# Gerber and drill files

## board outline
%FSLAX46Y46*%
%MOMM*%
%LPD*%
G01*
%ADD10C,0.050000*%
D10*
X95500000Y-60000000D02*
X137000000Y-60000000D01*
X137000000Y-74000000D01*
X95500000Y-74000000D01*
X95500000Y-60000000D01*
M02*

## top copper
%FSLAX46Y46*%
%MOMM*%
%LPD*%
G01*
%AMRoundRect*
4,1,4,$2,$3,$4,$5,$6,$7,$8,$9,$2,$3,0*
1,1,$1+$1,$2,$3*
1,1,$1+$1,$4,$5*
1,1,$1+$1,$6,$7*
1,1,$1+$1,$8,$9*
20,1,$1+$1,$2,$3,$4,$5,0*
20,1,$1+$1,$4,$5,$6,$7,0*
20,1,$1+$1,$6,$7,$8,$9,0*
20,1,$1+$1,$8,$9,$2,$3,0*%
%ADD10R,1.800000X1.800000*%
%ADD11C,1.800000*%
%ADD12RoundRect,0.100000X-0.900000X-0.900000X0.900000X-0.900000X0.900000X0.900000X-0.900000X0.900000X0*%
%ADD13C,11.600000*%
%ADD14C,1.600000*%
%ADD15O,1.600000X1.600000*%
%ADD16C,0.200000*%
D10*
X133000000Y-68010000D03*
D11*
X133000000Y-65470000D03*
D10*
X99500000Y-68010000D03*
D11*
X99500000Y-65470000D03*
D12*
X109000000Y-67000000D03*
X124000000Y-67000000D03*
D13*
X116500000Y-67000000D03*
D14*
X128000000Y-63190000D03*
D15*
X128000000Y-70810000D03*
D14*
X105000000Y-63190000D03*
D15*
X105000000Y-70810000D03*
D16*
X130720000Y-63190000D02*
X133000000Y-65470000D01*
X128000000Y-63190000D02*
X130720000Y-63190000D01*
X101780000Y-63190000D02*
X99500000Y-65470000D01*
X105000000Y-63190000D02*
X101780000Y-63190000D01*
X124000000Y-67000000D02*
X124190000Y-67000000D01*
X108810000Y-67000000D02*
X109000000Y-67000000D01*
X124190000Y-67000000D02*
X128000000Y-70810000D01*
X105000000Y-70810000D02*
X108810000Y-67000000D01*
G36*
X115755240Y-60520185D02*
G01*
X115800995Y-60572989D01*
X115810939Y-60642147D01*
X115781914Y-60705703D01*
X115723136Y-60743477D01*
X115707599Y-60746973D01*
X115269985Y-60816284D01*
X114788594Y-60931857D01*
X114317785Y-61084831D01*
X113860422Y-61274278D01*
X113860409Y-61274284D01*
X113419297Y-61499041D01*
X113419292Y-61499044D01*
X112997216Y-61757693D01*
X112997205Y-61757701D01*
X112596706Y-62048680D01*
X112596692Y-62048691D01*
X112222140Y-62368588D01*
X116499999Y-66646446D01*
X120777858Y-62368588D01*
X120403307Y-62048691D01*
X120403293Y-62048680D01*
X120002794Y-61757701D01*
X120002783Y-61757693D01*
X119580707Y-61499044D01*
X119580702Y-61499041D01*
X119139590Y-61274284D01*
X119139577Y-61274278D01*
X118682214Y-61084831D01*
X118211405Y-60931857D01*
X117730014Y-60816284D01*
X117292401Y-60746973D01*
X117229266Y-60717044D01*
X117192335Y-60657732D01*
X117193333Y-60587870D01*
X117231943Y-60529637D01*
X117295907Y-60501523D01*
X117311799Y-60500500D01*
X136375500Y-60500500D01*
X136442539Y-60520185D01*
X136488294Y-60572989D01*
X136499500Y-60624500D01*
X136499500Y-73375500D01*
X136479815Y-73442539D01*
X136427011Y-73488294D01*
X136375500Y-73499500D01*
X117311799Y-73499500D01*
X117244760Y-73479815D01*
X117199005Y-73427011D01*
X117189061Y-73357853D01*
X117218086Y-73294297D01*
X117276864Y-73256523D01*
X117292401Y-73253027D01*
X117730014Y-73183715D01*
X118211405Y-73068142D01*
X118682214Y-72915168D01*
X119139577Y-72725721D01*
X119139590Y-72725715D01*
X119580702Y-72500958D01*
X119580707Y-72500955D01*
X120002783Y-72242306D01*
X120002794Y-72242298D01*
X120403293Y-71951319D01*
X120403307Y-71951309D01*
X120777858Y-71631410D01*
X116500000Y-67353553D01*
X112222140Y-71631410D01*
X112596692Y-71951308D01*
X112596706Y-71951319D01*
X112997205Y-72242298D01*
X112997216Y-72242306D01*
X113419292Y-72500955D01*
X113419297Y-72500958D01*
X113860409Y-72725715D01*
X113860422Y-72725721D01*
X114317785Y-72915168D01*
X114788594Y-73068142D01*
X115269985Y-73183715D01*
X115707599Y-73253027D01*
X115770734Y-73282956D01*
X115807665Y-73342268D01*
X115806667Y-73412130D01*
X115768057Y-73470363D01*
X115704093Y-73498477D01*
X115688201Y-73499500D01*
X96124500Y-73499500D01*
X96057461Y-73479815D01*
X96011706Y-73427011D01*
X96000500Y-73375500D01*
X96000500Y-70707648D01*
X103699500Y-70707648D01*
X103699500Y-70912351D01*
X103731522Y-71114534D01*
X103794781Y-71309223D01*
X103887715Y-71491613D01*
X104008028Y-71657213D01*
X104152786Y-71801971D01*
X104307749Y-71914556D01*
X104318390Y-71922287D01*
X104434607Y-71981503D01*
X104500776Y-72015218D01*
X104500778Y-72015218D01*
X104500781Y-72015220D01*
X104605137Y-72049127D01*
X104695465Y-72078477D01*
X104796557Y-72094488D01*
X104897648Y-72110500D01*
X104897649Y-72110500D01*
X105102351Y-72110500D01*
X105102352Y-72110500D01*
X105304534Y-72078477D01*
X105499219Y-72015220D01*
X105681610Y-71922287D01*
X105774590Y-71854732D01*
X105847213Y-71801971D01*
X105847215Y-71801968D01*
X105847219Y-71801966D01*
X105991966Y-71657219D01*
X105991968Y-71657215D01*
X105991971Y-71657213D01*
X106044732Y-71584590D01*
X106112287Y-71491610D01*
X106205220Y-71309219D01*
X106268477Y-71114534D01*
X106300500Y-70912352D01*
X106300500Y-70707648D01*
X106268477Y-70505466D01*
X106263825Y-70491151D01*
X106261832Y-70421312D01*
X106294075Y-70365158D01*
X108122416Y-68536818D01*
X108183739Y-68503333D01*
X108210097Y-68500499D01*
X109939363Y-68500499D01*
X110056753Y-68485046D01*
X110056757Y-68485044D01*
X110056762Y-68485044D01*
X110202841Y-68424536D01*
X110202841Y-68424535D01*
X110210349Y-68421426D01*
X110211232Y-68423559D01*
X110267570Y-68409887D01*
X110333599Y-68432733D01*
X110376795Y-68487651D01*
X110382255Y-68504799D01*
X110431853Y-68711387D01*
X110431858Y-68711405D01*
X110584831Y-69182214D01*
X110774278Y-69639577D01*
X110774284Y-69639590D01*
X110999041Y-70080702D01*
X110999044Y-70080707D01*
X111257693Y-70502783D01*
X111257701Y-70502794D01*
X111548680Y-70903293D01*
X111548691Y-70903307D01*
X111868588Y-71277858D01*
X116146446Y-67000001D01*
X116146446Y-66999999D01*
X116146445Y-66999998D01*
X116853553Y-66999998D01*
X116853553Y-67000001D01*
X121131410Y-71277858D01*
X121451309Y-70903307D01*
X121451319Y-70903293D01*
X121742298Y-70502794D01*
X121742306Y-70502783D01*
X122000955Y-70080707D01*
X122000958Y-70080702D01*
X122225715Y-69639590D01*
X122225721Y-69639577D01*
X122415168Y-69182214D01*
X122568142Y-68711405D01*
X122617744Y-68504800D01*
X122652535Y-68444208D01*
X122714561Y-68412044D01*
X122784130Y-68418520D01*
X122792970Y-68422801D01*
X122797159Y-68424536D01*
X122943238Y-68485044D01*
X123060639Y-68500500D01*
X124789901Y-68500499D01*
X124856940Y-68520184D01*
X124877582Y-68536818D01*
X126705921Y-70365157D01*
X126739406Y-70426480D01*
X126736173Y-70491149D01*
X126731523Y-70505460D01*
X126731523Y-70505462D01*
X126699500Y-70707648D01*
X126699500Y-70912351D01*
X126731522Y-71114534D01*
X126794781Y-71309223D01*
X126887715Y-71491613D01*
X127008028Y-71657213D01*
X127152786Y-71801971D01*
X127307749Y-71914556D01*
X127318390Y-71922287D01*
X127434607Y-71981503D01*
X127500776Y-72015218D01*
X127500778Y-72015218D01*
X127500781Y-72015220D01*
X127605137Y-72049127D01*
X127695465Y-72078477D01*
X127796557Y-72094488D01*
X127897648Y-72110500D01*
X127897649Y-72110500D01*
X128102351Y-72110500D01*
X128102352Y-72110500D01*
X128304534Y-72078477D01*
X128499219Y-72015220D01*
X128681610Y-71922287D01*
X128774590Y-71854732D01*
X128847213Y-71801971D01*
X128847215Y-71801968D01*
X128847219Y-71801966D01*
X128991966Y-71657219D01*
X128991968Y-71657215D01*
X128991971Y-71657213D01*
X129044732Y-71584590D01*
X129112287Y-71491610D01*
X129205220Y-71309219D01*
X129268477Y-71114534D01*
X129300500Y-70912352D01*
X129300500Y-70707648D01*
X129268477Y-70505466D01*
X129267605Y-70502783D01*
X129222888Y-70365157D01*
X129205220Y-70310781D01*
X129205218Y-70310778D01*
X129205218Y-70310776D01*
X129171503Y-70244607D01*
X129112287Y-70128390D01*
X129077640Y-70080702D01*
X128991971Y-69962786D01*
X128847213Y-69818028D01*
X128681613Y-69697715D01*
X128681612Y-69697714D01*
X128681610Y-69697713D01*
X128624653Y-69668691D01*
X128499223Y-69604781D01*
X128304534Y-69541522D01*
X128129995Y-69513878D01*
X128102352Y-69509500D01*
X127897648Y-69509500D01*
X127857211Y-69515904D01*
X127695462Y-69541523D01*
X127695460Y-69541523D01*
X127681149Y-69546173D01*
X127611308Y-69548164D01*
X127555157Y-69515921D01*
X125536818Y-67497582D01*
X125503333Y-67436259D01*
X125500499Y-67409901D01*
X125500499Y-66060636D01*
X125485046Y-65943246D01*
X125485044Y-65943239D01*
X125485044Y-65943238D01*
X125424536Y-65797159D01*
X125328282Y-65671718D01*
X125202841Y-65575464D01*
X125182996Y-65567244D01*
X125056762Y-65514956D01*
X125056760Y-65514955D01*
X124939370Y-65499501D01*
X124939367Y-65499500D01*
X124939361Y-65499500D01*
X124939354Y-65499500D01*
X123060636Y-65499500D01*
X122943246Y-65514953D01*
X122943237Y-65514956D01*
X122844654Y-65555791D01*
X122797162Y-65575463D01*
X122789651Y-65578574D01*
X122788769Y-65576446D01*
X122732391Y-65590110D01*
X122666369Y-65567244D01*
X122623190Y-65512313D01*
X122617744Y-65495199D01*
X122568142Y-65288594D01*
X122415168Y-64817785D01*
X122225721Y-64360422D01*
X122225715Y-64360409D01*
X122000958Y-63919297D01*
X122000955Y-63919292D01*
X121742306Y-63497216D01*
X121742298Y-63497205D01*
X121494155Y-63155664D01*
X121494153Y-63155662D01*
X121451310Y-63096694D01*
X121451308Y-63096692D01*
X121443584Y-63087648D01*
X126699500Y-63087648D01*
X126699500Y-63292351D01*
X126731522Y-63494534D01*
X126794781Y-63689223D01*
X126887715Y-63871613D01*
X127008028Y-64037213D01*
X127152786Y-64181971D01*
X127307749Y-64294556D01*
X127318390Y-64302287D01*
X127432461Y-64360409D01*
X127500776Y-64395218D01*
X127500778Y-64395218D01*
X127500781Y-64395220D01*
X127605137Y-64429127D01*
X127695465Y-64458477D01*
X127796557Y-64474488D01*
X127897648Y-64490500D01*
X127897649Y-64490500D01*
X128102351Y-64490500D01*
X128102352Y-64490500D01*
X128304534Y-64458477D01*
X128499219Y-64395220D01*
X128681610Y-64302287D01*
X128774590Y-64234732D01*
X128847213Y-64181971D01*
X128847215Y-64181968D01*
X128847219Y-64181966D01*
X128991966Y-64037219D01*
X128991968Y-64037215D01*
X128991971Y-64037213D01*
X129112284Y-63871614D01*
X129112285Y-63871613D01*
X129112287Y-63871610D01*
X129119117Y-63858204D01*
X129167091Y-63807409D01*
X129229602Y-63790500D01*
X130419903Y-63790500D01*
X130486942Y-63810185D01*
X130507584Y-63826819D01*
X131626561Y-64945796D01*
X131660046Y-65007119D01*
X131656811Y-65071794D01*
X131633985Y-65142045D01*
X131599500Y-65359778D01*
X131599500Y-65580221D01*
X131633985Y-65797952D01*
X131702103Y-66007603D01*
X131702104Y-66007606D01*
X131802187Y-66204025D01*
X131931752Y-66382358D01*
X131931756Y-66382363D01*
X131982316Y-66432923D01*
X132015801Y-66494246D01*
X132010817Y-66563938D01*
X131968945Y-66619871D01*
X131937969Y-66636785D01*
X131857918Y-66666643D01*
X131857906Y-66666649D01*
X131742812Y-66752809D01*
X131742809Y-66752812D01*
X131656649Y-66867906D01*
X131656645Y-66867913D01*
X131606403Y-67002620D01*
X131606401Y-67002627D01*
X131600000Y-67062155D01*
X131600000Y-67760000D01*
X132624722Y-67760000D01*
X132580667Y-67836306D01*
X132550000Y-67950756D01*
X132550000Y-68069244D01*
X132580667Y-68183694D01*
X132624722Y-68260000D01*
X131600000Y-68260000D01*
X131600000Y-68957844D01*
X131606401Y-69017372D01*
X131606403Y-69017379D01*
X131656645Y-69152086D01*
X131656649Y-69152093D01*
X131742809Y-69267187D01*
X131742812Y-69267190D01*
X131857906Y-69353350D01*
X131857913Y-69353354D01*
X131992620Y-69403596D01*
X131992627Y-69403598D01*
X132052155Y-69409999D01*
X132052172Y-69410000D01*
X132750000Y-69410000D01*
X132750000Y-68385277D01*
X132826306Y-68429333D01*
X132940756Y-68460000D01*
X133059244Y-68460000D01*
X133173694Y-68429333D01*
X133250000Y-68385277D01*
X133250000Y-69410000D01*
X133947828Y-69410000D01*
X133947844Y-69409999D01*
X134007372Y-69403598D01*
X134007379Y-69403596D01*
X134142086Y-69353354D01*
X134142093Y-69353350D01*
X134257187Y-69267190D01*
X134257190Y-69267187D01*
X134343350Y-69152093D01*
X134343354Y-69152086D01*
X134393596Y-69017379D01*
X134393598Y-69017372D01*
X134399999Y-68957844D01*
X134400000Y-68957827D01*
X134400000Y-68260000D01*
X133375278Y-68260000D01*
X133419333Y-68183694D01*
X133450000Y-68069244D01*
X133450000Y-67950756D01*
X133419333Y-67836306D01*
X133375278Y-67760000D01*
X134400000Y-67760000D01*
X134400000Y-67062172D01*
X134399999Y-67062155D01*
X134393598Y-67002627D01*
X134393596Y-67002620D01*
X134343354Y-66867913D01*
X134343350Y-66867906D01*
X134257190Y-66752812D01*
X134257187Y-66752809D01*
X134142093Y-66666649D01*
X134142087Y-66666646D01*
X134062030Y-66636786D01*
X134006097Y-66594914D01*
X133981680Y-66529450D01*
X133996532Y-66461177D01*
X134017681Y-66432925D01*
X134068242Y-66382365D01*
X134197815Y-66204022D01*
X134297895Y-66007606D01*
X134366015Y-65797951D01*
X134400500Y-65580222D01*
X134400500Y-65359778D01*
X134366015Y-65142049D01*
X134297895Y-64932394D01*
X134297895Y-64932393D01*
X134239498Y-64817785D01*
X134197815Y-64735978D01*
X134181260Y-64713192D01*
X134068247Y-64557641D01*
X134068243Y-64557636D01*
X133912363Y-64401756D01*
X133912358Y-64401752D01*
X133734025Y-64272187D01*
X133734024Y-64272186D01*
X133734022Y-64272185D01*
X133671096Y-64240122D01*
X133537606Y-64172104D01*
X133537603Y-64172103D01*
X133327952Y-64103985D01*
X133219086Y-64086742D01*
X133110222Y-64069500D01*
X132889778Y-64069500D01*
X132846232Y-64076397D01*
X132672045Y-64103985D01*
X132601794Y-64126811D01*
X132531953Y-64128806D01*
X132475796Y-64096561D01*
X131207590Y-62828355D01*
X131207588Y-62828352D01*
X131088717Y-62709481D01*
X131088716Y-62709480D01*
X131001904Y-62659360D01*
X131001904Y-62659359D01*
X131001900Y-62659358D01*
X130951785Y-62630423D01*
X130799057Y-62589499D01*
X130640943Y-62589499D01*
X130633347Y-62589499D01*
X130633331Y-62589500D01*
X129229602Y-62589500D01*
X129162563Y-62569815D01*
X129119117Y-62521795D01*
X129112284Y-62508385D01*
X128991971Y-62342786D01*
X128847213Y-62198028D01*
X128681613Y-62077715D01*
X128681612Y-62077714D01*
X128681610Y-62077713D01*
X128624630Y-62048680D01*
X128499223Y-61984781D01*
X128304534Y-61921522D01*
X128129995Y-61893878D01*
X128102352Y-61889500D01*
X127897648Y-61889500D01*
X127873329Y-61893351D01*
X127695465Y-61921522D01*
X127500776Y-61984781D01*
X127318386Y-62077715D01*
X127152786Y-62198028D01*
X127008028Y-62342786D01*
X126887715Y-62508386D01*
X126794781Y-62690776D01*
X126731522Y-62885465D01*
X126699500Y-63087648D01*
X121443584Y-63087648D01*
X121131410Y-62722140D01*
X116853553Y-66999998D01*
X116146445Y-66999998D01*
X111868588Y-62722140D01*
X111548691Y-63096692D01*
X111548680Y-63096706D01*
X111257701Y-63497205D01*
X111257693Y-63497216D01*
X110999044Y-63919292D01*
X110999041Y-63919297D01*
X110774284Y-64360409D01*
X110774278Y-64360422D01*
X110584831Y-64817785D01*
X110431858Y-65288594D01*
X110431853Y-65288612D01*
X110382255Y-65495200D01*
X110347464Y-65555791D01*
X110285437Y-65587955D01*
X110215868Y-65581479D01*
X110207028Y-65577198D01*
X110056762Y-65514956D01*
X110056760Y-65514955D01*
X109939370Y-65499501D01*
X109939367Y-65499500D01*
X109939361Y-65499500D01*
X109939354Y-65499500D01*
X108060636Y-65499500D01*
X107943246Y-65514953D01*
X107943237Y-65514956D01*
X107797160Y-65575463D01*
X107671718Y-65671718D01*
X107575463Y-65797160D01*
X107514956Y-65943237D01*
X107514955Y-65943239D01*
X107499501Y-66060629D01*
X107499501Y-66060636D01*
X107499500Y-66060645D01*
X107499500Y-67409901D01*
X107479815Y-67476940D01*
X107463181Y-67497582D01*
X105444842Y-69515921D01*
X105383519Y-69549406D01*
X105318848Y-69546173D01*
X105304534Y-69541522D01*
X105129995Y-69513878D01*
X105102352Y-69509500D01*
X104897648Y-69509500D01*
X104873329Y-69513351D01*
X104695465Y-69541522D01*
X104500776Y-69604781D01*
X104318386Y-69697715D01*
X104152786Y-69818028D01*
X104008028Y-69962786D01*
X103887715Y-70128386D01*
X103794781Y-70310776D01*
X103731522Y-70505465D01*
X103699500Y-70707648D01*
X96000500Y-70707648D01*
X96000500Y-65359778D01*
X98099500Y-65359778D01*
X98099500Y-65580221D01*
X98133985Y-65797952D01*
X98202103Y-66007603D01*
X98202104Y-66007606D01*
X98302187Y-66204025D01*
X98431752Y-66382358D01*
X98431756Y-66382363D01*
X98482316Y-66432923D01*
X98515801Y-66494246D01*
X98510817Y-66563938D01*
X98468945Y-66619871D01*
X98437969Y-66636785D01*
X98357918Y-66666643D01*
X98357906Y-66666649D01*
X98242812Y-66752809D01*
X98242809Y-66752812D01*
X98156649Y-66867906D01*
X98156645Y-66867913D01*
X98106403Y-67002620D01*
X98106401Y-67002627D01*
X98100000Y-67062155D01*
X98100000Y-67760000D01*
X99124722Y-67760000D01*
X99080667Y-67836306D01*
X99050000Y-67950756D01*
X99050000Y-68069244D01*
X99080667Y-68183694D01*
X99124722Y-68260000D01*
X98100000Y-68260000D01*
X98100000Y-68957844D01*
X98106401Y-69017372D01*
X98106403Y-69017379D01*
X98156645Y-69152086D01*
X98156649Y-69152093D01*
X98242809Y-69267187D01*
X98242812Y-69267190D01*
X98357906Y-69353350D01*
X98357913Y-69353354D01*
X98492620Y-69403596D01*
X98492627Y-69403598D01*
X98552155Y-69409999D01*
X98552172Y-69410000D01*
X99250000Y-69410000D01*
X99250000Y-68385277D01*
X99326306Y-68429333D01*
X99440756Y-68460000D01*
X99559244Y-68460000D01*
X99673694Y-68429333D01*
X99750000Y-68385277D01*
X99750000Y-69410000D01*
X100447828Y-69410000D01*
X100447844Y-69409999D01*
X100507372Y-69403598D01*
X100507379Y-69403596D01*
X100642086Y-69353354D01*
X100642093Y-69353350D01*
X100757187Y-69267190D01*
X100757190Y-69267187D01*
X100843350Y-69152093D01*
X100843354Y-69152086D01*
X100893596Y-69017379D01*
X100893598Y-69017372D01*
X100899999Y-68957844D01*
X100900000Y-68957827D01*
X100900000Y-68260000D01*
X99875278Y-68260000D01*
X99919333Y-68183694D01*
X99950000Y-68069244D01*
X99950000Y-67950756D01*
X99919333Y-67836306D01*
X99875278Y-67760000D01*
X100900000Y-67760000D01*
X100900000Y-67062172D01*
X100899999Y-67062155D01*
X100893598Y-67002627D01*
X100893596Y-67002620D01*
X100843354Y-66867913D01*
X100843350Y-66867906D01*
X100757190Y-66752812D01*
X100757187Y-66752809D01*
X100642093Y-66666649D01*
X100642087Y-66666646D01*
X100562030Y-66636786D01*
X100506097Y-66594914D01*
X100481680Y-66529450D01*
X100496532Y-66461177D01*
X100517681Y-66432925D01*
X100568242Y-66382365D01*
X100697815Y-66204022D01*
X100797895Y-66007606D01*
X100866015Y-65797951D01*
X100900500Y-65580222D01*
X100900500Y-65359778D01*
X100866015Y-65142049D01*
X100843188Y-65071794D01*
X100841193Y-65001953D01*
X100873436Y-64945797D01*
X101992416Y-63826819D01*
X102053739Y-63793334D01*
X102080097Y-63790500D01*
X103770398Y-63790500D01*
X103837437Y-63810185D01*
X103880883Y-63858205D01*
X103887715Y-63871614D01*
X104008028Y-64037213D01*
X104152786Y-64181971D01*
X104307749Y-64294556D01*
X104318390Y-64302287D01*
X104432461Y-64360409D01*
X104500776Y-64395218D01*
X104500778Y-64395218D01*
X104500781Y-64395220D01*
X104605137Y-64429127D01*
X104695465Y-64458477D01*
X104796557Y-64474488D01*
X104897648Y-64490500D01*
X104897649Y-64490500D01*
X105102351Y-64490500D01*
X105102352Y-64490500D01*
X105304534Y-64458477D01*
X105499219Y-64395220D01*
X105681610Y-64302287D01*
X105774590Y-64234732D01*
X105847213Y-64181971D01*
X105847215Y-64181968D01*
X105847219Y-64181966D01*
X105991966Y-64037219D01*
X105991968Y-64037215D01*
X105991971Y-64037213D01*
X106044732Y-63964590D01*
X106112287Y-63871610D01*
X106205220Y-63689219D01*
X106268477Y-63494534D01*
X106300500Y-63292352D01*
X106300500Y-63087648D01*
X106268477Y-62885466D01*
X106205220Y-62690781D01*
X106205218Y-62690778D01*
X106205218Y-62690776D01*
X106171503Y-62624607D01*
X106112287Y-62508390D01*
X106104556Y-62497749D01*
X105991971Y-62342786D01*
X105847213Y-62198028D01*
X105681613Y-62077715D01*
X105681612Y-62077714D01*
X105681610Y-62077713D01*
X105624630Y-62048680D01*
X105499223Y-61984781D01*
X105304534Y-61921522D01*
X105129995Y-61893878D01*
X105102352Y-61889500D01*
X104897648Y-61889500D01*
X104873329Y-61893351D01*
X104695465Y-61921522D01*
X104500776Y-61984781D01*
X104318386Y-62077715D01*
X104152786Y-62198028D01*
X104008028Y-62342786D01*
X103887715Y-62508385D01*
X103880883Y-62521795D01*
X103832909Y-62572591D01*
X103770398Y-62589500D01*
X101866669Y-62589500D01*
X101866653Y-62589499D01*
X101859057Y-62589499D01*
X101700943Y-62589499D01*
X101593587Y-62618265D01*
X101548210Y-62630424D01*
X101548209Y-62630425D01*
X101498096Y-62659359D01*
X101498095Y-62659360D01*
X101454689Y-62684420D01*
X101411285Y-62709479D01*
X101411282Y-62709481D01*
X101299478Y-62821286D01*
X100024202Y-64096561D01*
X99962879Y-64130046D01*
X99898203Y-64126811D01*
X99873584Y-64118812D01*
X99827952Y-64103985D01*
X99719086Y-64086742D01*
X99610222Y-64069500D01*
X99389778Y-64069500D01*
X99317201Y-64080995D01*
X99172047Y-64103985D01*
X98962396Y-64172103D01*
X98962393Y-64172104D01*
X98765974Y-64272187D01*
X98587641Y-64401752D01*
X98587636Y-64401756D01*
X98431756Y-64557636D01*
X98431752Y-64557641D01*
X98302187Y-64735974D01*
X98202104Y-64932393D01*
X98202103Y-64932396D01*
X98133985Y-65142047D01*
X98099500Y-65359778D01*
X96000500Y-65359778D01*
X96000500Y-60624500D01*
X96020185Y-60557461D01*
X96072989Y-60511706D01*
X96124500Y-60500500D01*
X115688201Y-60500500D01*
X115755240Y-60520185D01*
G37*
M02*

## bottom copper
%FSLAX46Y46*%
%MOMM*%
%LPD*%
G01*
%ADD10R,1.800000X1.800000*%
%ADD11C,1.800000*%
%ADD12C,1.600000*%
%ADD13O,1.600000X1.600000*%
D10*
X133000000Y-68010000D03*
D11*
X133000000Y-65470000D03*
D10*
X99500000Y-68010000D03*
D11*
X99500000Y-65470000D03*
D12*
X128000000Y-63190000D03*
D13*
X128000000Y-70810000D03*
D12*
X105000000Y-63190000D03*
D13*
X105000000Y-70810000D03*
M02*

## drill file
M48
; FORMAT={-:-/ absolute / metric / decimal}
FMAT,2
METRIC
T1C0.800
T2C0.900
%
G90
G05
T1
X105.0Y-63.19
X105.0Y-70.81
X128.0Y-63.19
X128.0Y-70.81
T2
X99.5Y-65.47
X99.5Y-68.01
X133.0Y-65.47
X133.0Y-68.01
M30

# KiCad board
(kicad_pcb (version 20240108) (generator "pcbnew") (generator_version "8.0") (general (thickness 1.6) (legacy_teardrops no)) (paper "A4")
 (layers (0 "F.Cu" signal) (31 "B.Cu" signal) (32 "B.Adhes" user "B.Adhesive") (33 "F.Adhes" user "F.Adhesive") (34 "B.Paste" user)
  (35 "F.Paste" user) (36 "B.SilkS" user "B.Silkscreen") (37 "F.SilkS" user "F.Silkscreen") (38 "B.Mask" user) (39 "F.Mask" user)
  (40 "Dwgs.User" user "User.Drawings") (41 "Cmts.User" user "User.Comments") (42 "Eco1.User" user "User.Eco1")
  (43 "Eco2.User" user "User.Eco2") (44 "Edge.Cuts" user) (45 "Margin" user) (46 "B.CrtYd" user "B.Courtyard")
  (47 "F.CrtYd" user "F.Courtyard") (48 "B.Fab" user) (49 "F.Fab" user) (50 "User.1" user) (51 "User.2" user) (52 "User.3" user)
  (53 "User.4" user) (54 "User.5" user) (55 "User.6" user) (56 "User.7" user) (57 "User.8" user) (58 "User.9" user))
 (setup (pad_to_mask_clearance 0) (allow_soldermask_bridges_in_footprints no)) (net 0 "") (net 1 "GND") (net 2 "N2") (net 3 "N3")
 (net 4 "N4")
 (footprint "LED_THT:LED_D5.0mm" (layer "F.Cu") (at 133 68.01 90)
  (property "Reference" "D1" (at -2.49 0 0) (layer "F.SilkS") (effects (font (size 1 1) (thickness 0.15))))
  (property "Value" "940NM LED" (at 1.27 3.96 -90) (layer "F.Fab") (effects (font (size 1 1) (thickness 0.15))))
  (pad "1" thru_hole rect (at 0 0 90) (size 1.8 1.8) (drill 0.9) (layers "*.Cu" "*.Mask") (remove_unused_layers no) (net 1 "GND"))
  (pad "2" thru_hole circle (at 2.54 0 90) (size 1.8 1.8) (drill 0.9) (layers "*.Cu" "*.Mask") (remove_unused_layers no) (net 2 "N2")))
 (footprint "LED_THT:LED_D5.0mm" (layer "F.Cu") (at 99.5 68.01 90)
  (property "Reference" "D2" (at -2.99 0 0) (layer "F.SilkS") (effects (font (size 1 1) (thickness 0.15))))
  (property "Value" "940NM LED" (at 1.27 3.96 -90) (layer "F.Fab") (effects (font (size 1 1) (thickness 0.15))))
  (pad "1" thru_hole rect (at 0 0 90) (size 1.8 1.8) (drill 0.9) (layers "*.Cu" "*.Mask") (remove_unused_layers no) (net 1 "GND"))
  (pad "2" thru_hole circle (at 2.54 0 90) (size 1.8 1.8) (drill 0.9) (layers "*.Cu" "*.Mask") (remove_unused_layers no) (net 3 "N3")))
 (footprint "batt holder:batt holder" (layer "F.Cu") (at 116.5 67)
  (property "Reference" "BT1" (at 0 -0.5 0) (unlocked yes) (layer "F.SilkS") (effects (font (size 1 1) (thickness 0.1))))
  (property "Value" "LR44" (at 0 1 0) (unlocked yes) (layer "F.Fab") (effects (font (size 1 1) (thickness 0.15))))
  (pad "1" smd roundrect (at -7.5 0) (size 2 2) (layers "F.Cu" "F.Paste" "F.Mask") (roundrect_rratio 0.05) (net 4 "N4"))
  (pad "1" smd roundrect (at 7.5 0) (size 2 2) (layers "F.Cu" "F.Paste" "F.Mask") (roundrect_rratio 0.05) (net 4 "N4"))
  (pad "2" smd circle (at 0 0) (size 11.6 11.6) (layers "F.Cu" "F.Paste" "F.Mask") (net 1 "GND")))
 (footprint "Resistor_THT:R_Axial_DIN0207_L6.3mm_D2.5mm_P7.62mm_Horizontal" (layer "F.Cu") (at 128 63.19 -90)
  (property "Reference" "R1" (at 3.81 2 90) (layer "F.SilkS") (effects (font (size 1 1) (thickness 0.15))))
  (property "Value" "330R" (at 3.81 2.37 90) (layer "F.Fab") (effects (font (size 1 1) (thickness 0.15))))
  (pad "1" thru_hole circle (at 0 0 270) (size 1.6 1.6) (drill 0.8) (layers "*.Cu" "*.Mask") (remove_unused_layers no) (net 2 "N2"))
  (pad "2" thru_hole oval (at 7.62 0 270) (size 1.6 1.6) (drill 0.8) (layers "*.Cu" "*.Mask") (remove_unused_layers no) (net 4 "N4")))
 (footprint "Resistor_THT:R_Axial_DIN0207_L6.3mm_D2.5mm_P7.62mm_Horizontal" (layer "F.Cu") (at 105 63.19 -90)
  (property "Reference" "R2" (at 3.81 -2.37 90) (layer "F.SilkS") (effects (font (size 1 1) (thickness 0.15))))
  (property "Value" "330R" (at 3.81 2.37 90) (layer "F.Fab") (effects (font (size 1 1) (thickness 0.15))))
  (pad "1" thru_hole circle (at 0 0 270) (size 1.6 1.6) (drill 0.8) (layers "*.Cu" "*.Mask") (remove_unused_layers no) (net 3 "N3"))
  (pad "2" thru_hole oval (at 7.62 0 270) (size 1.6 1.6) (drill 0.8) (layers "*.Cu" "*.Mask") (remove_unused_layers no) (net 4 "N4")))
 (gr_rect (start 95.5 60) (end 137 74) (stroke (width 0.05) (type default)) (fill none) (layer "Edge.Cuts"))
 (segment (start 130.72 63.19) (end 133 65.47) (width 0.2) (layer "F.Cu") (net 2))
 (segment (start 128 63.19) (end 130.72 63.19) (width 0.2) (layer "F.Cu") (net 2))
 (segment (start 101.78 63.19) (end 99.5 65.47) (width 0.2) (layer "F.Cu") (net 3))
 (segment (start 105 63.19) (end 101.78 63.19) (width 0.2) (layer "F.Cu") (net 3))
 (segment (start 124 67) (end 124.19 67) (width 0.2) (layer "F.Cu") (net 4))
 (segment (start 108.81 67) (end 109 67) (width 0.2) (layer "F.Cu") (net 4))
 (segment (start 124.19 67) (end 128 70.81) (width 0.2) (layer "F.Cu") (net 4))
 (segment (start 105 70.81) (end 108.81 67) (width 0.2) (layer "F.Cu") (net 4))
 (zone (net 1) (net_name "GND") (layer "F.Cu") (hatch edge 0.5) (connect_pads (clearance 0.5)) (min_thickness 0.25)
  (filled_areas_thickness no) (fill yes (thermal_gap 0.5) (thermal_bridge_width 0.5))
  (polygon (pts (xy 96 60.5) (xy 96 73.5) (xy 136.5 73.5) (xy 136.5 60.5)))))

